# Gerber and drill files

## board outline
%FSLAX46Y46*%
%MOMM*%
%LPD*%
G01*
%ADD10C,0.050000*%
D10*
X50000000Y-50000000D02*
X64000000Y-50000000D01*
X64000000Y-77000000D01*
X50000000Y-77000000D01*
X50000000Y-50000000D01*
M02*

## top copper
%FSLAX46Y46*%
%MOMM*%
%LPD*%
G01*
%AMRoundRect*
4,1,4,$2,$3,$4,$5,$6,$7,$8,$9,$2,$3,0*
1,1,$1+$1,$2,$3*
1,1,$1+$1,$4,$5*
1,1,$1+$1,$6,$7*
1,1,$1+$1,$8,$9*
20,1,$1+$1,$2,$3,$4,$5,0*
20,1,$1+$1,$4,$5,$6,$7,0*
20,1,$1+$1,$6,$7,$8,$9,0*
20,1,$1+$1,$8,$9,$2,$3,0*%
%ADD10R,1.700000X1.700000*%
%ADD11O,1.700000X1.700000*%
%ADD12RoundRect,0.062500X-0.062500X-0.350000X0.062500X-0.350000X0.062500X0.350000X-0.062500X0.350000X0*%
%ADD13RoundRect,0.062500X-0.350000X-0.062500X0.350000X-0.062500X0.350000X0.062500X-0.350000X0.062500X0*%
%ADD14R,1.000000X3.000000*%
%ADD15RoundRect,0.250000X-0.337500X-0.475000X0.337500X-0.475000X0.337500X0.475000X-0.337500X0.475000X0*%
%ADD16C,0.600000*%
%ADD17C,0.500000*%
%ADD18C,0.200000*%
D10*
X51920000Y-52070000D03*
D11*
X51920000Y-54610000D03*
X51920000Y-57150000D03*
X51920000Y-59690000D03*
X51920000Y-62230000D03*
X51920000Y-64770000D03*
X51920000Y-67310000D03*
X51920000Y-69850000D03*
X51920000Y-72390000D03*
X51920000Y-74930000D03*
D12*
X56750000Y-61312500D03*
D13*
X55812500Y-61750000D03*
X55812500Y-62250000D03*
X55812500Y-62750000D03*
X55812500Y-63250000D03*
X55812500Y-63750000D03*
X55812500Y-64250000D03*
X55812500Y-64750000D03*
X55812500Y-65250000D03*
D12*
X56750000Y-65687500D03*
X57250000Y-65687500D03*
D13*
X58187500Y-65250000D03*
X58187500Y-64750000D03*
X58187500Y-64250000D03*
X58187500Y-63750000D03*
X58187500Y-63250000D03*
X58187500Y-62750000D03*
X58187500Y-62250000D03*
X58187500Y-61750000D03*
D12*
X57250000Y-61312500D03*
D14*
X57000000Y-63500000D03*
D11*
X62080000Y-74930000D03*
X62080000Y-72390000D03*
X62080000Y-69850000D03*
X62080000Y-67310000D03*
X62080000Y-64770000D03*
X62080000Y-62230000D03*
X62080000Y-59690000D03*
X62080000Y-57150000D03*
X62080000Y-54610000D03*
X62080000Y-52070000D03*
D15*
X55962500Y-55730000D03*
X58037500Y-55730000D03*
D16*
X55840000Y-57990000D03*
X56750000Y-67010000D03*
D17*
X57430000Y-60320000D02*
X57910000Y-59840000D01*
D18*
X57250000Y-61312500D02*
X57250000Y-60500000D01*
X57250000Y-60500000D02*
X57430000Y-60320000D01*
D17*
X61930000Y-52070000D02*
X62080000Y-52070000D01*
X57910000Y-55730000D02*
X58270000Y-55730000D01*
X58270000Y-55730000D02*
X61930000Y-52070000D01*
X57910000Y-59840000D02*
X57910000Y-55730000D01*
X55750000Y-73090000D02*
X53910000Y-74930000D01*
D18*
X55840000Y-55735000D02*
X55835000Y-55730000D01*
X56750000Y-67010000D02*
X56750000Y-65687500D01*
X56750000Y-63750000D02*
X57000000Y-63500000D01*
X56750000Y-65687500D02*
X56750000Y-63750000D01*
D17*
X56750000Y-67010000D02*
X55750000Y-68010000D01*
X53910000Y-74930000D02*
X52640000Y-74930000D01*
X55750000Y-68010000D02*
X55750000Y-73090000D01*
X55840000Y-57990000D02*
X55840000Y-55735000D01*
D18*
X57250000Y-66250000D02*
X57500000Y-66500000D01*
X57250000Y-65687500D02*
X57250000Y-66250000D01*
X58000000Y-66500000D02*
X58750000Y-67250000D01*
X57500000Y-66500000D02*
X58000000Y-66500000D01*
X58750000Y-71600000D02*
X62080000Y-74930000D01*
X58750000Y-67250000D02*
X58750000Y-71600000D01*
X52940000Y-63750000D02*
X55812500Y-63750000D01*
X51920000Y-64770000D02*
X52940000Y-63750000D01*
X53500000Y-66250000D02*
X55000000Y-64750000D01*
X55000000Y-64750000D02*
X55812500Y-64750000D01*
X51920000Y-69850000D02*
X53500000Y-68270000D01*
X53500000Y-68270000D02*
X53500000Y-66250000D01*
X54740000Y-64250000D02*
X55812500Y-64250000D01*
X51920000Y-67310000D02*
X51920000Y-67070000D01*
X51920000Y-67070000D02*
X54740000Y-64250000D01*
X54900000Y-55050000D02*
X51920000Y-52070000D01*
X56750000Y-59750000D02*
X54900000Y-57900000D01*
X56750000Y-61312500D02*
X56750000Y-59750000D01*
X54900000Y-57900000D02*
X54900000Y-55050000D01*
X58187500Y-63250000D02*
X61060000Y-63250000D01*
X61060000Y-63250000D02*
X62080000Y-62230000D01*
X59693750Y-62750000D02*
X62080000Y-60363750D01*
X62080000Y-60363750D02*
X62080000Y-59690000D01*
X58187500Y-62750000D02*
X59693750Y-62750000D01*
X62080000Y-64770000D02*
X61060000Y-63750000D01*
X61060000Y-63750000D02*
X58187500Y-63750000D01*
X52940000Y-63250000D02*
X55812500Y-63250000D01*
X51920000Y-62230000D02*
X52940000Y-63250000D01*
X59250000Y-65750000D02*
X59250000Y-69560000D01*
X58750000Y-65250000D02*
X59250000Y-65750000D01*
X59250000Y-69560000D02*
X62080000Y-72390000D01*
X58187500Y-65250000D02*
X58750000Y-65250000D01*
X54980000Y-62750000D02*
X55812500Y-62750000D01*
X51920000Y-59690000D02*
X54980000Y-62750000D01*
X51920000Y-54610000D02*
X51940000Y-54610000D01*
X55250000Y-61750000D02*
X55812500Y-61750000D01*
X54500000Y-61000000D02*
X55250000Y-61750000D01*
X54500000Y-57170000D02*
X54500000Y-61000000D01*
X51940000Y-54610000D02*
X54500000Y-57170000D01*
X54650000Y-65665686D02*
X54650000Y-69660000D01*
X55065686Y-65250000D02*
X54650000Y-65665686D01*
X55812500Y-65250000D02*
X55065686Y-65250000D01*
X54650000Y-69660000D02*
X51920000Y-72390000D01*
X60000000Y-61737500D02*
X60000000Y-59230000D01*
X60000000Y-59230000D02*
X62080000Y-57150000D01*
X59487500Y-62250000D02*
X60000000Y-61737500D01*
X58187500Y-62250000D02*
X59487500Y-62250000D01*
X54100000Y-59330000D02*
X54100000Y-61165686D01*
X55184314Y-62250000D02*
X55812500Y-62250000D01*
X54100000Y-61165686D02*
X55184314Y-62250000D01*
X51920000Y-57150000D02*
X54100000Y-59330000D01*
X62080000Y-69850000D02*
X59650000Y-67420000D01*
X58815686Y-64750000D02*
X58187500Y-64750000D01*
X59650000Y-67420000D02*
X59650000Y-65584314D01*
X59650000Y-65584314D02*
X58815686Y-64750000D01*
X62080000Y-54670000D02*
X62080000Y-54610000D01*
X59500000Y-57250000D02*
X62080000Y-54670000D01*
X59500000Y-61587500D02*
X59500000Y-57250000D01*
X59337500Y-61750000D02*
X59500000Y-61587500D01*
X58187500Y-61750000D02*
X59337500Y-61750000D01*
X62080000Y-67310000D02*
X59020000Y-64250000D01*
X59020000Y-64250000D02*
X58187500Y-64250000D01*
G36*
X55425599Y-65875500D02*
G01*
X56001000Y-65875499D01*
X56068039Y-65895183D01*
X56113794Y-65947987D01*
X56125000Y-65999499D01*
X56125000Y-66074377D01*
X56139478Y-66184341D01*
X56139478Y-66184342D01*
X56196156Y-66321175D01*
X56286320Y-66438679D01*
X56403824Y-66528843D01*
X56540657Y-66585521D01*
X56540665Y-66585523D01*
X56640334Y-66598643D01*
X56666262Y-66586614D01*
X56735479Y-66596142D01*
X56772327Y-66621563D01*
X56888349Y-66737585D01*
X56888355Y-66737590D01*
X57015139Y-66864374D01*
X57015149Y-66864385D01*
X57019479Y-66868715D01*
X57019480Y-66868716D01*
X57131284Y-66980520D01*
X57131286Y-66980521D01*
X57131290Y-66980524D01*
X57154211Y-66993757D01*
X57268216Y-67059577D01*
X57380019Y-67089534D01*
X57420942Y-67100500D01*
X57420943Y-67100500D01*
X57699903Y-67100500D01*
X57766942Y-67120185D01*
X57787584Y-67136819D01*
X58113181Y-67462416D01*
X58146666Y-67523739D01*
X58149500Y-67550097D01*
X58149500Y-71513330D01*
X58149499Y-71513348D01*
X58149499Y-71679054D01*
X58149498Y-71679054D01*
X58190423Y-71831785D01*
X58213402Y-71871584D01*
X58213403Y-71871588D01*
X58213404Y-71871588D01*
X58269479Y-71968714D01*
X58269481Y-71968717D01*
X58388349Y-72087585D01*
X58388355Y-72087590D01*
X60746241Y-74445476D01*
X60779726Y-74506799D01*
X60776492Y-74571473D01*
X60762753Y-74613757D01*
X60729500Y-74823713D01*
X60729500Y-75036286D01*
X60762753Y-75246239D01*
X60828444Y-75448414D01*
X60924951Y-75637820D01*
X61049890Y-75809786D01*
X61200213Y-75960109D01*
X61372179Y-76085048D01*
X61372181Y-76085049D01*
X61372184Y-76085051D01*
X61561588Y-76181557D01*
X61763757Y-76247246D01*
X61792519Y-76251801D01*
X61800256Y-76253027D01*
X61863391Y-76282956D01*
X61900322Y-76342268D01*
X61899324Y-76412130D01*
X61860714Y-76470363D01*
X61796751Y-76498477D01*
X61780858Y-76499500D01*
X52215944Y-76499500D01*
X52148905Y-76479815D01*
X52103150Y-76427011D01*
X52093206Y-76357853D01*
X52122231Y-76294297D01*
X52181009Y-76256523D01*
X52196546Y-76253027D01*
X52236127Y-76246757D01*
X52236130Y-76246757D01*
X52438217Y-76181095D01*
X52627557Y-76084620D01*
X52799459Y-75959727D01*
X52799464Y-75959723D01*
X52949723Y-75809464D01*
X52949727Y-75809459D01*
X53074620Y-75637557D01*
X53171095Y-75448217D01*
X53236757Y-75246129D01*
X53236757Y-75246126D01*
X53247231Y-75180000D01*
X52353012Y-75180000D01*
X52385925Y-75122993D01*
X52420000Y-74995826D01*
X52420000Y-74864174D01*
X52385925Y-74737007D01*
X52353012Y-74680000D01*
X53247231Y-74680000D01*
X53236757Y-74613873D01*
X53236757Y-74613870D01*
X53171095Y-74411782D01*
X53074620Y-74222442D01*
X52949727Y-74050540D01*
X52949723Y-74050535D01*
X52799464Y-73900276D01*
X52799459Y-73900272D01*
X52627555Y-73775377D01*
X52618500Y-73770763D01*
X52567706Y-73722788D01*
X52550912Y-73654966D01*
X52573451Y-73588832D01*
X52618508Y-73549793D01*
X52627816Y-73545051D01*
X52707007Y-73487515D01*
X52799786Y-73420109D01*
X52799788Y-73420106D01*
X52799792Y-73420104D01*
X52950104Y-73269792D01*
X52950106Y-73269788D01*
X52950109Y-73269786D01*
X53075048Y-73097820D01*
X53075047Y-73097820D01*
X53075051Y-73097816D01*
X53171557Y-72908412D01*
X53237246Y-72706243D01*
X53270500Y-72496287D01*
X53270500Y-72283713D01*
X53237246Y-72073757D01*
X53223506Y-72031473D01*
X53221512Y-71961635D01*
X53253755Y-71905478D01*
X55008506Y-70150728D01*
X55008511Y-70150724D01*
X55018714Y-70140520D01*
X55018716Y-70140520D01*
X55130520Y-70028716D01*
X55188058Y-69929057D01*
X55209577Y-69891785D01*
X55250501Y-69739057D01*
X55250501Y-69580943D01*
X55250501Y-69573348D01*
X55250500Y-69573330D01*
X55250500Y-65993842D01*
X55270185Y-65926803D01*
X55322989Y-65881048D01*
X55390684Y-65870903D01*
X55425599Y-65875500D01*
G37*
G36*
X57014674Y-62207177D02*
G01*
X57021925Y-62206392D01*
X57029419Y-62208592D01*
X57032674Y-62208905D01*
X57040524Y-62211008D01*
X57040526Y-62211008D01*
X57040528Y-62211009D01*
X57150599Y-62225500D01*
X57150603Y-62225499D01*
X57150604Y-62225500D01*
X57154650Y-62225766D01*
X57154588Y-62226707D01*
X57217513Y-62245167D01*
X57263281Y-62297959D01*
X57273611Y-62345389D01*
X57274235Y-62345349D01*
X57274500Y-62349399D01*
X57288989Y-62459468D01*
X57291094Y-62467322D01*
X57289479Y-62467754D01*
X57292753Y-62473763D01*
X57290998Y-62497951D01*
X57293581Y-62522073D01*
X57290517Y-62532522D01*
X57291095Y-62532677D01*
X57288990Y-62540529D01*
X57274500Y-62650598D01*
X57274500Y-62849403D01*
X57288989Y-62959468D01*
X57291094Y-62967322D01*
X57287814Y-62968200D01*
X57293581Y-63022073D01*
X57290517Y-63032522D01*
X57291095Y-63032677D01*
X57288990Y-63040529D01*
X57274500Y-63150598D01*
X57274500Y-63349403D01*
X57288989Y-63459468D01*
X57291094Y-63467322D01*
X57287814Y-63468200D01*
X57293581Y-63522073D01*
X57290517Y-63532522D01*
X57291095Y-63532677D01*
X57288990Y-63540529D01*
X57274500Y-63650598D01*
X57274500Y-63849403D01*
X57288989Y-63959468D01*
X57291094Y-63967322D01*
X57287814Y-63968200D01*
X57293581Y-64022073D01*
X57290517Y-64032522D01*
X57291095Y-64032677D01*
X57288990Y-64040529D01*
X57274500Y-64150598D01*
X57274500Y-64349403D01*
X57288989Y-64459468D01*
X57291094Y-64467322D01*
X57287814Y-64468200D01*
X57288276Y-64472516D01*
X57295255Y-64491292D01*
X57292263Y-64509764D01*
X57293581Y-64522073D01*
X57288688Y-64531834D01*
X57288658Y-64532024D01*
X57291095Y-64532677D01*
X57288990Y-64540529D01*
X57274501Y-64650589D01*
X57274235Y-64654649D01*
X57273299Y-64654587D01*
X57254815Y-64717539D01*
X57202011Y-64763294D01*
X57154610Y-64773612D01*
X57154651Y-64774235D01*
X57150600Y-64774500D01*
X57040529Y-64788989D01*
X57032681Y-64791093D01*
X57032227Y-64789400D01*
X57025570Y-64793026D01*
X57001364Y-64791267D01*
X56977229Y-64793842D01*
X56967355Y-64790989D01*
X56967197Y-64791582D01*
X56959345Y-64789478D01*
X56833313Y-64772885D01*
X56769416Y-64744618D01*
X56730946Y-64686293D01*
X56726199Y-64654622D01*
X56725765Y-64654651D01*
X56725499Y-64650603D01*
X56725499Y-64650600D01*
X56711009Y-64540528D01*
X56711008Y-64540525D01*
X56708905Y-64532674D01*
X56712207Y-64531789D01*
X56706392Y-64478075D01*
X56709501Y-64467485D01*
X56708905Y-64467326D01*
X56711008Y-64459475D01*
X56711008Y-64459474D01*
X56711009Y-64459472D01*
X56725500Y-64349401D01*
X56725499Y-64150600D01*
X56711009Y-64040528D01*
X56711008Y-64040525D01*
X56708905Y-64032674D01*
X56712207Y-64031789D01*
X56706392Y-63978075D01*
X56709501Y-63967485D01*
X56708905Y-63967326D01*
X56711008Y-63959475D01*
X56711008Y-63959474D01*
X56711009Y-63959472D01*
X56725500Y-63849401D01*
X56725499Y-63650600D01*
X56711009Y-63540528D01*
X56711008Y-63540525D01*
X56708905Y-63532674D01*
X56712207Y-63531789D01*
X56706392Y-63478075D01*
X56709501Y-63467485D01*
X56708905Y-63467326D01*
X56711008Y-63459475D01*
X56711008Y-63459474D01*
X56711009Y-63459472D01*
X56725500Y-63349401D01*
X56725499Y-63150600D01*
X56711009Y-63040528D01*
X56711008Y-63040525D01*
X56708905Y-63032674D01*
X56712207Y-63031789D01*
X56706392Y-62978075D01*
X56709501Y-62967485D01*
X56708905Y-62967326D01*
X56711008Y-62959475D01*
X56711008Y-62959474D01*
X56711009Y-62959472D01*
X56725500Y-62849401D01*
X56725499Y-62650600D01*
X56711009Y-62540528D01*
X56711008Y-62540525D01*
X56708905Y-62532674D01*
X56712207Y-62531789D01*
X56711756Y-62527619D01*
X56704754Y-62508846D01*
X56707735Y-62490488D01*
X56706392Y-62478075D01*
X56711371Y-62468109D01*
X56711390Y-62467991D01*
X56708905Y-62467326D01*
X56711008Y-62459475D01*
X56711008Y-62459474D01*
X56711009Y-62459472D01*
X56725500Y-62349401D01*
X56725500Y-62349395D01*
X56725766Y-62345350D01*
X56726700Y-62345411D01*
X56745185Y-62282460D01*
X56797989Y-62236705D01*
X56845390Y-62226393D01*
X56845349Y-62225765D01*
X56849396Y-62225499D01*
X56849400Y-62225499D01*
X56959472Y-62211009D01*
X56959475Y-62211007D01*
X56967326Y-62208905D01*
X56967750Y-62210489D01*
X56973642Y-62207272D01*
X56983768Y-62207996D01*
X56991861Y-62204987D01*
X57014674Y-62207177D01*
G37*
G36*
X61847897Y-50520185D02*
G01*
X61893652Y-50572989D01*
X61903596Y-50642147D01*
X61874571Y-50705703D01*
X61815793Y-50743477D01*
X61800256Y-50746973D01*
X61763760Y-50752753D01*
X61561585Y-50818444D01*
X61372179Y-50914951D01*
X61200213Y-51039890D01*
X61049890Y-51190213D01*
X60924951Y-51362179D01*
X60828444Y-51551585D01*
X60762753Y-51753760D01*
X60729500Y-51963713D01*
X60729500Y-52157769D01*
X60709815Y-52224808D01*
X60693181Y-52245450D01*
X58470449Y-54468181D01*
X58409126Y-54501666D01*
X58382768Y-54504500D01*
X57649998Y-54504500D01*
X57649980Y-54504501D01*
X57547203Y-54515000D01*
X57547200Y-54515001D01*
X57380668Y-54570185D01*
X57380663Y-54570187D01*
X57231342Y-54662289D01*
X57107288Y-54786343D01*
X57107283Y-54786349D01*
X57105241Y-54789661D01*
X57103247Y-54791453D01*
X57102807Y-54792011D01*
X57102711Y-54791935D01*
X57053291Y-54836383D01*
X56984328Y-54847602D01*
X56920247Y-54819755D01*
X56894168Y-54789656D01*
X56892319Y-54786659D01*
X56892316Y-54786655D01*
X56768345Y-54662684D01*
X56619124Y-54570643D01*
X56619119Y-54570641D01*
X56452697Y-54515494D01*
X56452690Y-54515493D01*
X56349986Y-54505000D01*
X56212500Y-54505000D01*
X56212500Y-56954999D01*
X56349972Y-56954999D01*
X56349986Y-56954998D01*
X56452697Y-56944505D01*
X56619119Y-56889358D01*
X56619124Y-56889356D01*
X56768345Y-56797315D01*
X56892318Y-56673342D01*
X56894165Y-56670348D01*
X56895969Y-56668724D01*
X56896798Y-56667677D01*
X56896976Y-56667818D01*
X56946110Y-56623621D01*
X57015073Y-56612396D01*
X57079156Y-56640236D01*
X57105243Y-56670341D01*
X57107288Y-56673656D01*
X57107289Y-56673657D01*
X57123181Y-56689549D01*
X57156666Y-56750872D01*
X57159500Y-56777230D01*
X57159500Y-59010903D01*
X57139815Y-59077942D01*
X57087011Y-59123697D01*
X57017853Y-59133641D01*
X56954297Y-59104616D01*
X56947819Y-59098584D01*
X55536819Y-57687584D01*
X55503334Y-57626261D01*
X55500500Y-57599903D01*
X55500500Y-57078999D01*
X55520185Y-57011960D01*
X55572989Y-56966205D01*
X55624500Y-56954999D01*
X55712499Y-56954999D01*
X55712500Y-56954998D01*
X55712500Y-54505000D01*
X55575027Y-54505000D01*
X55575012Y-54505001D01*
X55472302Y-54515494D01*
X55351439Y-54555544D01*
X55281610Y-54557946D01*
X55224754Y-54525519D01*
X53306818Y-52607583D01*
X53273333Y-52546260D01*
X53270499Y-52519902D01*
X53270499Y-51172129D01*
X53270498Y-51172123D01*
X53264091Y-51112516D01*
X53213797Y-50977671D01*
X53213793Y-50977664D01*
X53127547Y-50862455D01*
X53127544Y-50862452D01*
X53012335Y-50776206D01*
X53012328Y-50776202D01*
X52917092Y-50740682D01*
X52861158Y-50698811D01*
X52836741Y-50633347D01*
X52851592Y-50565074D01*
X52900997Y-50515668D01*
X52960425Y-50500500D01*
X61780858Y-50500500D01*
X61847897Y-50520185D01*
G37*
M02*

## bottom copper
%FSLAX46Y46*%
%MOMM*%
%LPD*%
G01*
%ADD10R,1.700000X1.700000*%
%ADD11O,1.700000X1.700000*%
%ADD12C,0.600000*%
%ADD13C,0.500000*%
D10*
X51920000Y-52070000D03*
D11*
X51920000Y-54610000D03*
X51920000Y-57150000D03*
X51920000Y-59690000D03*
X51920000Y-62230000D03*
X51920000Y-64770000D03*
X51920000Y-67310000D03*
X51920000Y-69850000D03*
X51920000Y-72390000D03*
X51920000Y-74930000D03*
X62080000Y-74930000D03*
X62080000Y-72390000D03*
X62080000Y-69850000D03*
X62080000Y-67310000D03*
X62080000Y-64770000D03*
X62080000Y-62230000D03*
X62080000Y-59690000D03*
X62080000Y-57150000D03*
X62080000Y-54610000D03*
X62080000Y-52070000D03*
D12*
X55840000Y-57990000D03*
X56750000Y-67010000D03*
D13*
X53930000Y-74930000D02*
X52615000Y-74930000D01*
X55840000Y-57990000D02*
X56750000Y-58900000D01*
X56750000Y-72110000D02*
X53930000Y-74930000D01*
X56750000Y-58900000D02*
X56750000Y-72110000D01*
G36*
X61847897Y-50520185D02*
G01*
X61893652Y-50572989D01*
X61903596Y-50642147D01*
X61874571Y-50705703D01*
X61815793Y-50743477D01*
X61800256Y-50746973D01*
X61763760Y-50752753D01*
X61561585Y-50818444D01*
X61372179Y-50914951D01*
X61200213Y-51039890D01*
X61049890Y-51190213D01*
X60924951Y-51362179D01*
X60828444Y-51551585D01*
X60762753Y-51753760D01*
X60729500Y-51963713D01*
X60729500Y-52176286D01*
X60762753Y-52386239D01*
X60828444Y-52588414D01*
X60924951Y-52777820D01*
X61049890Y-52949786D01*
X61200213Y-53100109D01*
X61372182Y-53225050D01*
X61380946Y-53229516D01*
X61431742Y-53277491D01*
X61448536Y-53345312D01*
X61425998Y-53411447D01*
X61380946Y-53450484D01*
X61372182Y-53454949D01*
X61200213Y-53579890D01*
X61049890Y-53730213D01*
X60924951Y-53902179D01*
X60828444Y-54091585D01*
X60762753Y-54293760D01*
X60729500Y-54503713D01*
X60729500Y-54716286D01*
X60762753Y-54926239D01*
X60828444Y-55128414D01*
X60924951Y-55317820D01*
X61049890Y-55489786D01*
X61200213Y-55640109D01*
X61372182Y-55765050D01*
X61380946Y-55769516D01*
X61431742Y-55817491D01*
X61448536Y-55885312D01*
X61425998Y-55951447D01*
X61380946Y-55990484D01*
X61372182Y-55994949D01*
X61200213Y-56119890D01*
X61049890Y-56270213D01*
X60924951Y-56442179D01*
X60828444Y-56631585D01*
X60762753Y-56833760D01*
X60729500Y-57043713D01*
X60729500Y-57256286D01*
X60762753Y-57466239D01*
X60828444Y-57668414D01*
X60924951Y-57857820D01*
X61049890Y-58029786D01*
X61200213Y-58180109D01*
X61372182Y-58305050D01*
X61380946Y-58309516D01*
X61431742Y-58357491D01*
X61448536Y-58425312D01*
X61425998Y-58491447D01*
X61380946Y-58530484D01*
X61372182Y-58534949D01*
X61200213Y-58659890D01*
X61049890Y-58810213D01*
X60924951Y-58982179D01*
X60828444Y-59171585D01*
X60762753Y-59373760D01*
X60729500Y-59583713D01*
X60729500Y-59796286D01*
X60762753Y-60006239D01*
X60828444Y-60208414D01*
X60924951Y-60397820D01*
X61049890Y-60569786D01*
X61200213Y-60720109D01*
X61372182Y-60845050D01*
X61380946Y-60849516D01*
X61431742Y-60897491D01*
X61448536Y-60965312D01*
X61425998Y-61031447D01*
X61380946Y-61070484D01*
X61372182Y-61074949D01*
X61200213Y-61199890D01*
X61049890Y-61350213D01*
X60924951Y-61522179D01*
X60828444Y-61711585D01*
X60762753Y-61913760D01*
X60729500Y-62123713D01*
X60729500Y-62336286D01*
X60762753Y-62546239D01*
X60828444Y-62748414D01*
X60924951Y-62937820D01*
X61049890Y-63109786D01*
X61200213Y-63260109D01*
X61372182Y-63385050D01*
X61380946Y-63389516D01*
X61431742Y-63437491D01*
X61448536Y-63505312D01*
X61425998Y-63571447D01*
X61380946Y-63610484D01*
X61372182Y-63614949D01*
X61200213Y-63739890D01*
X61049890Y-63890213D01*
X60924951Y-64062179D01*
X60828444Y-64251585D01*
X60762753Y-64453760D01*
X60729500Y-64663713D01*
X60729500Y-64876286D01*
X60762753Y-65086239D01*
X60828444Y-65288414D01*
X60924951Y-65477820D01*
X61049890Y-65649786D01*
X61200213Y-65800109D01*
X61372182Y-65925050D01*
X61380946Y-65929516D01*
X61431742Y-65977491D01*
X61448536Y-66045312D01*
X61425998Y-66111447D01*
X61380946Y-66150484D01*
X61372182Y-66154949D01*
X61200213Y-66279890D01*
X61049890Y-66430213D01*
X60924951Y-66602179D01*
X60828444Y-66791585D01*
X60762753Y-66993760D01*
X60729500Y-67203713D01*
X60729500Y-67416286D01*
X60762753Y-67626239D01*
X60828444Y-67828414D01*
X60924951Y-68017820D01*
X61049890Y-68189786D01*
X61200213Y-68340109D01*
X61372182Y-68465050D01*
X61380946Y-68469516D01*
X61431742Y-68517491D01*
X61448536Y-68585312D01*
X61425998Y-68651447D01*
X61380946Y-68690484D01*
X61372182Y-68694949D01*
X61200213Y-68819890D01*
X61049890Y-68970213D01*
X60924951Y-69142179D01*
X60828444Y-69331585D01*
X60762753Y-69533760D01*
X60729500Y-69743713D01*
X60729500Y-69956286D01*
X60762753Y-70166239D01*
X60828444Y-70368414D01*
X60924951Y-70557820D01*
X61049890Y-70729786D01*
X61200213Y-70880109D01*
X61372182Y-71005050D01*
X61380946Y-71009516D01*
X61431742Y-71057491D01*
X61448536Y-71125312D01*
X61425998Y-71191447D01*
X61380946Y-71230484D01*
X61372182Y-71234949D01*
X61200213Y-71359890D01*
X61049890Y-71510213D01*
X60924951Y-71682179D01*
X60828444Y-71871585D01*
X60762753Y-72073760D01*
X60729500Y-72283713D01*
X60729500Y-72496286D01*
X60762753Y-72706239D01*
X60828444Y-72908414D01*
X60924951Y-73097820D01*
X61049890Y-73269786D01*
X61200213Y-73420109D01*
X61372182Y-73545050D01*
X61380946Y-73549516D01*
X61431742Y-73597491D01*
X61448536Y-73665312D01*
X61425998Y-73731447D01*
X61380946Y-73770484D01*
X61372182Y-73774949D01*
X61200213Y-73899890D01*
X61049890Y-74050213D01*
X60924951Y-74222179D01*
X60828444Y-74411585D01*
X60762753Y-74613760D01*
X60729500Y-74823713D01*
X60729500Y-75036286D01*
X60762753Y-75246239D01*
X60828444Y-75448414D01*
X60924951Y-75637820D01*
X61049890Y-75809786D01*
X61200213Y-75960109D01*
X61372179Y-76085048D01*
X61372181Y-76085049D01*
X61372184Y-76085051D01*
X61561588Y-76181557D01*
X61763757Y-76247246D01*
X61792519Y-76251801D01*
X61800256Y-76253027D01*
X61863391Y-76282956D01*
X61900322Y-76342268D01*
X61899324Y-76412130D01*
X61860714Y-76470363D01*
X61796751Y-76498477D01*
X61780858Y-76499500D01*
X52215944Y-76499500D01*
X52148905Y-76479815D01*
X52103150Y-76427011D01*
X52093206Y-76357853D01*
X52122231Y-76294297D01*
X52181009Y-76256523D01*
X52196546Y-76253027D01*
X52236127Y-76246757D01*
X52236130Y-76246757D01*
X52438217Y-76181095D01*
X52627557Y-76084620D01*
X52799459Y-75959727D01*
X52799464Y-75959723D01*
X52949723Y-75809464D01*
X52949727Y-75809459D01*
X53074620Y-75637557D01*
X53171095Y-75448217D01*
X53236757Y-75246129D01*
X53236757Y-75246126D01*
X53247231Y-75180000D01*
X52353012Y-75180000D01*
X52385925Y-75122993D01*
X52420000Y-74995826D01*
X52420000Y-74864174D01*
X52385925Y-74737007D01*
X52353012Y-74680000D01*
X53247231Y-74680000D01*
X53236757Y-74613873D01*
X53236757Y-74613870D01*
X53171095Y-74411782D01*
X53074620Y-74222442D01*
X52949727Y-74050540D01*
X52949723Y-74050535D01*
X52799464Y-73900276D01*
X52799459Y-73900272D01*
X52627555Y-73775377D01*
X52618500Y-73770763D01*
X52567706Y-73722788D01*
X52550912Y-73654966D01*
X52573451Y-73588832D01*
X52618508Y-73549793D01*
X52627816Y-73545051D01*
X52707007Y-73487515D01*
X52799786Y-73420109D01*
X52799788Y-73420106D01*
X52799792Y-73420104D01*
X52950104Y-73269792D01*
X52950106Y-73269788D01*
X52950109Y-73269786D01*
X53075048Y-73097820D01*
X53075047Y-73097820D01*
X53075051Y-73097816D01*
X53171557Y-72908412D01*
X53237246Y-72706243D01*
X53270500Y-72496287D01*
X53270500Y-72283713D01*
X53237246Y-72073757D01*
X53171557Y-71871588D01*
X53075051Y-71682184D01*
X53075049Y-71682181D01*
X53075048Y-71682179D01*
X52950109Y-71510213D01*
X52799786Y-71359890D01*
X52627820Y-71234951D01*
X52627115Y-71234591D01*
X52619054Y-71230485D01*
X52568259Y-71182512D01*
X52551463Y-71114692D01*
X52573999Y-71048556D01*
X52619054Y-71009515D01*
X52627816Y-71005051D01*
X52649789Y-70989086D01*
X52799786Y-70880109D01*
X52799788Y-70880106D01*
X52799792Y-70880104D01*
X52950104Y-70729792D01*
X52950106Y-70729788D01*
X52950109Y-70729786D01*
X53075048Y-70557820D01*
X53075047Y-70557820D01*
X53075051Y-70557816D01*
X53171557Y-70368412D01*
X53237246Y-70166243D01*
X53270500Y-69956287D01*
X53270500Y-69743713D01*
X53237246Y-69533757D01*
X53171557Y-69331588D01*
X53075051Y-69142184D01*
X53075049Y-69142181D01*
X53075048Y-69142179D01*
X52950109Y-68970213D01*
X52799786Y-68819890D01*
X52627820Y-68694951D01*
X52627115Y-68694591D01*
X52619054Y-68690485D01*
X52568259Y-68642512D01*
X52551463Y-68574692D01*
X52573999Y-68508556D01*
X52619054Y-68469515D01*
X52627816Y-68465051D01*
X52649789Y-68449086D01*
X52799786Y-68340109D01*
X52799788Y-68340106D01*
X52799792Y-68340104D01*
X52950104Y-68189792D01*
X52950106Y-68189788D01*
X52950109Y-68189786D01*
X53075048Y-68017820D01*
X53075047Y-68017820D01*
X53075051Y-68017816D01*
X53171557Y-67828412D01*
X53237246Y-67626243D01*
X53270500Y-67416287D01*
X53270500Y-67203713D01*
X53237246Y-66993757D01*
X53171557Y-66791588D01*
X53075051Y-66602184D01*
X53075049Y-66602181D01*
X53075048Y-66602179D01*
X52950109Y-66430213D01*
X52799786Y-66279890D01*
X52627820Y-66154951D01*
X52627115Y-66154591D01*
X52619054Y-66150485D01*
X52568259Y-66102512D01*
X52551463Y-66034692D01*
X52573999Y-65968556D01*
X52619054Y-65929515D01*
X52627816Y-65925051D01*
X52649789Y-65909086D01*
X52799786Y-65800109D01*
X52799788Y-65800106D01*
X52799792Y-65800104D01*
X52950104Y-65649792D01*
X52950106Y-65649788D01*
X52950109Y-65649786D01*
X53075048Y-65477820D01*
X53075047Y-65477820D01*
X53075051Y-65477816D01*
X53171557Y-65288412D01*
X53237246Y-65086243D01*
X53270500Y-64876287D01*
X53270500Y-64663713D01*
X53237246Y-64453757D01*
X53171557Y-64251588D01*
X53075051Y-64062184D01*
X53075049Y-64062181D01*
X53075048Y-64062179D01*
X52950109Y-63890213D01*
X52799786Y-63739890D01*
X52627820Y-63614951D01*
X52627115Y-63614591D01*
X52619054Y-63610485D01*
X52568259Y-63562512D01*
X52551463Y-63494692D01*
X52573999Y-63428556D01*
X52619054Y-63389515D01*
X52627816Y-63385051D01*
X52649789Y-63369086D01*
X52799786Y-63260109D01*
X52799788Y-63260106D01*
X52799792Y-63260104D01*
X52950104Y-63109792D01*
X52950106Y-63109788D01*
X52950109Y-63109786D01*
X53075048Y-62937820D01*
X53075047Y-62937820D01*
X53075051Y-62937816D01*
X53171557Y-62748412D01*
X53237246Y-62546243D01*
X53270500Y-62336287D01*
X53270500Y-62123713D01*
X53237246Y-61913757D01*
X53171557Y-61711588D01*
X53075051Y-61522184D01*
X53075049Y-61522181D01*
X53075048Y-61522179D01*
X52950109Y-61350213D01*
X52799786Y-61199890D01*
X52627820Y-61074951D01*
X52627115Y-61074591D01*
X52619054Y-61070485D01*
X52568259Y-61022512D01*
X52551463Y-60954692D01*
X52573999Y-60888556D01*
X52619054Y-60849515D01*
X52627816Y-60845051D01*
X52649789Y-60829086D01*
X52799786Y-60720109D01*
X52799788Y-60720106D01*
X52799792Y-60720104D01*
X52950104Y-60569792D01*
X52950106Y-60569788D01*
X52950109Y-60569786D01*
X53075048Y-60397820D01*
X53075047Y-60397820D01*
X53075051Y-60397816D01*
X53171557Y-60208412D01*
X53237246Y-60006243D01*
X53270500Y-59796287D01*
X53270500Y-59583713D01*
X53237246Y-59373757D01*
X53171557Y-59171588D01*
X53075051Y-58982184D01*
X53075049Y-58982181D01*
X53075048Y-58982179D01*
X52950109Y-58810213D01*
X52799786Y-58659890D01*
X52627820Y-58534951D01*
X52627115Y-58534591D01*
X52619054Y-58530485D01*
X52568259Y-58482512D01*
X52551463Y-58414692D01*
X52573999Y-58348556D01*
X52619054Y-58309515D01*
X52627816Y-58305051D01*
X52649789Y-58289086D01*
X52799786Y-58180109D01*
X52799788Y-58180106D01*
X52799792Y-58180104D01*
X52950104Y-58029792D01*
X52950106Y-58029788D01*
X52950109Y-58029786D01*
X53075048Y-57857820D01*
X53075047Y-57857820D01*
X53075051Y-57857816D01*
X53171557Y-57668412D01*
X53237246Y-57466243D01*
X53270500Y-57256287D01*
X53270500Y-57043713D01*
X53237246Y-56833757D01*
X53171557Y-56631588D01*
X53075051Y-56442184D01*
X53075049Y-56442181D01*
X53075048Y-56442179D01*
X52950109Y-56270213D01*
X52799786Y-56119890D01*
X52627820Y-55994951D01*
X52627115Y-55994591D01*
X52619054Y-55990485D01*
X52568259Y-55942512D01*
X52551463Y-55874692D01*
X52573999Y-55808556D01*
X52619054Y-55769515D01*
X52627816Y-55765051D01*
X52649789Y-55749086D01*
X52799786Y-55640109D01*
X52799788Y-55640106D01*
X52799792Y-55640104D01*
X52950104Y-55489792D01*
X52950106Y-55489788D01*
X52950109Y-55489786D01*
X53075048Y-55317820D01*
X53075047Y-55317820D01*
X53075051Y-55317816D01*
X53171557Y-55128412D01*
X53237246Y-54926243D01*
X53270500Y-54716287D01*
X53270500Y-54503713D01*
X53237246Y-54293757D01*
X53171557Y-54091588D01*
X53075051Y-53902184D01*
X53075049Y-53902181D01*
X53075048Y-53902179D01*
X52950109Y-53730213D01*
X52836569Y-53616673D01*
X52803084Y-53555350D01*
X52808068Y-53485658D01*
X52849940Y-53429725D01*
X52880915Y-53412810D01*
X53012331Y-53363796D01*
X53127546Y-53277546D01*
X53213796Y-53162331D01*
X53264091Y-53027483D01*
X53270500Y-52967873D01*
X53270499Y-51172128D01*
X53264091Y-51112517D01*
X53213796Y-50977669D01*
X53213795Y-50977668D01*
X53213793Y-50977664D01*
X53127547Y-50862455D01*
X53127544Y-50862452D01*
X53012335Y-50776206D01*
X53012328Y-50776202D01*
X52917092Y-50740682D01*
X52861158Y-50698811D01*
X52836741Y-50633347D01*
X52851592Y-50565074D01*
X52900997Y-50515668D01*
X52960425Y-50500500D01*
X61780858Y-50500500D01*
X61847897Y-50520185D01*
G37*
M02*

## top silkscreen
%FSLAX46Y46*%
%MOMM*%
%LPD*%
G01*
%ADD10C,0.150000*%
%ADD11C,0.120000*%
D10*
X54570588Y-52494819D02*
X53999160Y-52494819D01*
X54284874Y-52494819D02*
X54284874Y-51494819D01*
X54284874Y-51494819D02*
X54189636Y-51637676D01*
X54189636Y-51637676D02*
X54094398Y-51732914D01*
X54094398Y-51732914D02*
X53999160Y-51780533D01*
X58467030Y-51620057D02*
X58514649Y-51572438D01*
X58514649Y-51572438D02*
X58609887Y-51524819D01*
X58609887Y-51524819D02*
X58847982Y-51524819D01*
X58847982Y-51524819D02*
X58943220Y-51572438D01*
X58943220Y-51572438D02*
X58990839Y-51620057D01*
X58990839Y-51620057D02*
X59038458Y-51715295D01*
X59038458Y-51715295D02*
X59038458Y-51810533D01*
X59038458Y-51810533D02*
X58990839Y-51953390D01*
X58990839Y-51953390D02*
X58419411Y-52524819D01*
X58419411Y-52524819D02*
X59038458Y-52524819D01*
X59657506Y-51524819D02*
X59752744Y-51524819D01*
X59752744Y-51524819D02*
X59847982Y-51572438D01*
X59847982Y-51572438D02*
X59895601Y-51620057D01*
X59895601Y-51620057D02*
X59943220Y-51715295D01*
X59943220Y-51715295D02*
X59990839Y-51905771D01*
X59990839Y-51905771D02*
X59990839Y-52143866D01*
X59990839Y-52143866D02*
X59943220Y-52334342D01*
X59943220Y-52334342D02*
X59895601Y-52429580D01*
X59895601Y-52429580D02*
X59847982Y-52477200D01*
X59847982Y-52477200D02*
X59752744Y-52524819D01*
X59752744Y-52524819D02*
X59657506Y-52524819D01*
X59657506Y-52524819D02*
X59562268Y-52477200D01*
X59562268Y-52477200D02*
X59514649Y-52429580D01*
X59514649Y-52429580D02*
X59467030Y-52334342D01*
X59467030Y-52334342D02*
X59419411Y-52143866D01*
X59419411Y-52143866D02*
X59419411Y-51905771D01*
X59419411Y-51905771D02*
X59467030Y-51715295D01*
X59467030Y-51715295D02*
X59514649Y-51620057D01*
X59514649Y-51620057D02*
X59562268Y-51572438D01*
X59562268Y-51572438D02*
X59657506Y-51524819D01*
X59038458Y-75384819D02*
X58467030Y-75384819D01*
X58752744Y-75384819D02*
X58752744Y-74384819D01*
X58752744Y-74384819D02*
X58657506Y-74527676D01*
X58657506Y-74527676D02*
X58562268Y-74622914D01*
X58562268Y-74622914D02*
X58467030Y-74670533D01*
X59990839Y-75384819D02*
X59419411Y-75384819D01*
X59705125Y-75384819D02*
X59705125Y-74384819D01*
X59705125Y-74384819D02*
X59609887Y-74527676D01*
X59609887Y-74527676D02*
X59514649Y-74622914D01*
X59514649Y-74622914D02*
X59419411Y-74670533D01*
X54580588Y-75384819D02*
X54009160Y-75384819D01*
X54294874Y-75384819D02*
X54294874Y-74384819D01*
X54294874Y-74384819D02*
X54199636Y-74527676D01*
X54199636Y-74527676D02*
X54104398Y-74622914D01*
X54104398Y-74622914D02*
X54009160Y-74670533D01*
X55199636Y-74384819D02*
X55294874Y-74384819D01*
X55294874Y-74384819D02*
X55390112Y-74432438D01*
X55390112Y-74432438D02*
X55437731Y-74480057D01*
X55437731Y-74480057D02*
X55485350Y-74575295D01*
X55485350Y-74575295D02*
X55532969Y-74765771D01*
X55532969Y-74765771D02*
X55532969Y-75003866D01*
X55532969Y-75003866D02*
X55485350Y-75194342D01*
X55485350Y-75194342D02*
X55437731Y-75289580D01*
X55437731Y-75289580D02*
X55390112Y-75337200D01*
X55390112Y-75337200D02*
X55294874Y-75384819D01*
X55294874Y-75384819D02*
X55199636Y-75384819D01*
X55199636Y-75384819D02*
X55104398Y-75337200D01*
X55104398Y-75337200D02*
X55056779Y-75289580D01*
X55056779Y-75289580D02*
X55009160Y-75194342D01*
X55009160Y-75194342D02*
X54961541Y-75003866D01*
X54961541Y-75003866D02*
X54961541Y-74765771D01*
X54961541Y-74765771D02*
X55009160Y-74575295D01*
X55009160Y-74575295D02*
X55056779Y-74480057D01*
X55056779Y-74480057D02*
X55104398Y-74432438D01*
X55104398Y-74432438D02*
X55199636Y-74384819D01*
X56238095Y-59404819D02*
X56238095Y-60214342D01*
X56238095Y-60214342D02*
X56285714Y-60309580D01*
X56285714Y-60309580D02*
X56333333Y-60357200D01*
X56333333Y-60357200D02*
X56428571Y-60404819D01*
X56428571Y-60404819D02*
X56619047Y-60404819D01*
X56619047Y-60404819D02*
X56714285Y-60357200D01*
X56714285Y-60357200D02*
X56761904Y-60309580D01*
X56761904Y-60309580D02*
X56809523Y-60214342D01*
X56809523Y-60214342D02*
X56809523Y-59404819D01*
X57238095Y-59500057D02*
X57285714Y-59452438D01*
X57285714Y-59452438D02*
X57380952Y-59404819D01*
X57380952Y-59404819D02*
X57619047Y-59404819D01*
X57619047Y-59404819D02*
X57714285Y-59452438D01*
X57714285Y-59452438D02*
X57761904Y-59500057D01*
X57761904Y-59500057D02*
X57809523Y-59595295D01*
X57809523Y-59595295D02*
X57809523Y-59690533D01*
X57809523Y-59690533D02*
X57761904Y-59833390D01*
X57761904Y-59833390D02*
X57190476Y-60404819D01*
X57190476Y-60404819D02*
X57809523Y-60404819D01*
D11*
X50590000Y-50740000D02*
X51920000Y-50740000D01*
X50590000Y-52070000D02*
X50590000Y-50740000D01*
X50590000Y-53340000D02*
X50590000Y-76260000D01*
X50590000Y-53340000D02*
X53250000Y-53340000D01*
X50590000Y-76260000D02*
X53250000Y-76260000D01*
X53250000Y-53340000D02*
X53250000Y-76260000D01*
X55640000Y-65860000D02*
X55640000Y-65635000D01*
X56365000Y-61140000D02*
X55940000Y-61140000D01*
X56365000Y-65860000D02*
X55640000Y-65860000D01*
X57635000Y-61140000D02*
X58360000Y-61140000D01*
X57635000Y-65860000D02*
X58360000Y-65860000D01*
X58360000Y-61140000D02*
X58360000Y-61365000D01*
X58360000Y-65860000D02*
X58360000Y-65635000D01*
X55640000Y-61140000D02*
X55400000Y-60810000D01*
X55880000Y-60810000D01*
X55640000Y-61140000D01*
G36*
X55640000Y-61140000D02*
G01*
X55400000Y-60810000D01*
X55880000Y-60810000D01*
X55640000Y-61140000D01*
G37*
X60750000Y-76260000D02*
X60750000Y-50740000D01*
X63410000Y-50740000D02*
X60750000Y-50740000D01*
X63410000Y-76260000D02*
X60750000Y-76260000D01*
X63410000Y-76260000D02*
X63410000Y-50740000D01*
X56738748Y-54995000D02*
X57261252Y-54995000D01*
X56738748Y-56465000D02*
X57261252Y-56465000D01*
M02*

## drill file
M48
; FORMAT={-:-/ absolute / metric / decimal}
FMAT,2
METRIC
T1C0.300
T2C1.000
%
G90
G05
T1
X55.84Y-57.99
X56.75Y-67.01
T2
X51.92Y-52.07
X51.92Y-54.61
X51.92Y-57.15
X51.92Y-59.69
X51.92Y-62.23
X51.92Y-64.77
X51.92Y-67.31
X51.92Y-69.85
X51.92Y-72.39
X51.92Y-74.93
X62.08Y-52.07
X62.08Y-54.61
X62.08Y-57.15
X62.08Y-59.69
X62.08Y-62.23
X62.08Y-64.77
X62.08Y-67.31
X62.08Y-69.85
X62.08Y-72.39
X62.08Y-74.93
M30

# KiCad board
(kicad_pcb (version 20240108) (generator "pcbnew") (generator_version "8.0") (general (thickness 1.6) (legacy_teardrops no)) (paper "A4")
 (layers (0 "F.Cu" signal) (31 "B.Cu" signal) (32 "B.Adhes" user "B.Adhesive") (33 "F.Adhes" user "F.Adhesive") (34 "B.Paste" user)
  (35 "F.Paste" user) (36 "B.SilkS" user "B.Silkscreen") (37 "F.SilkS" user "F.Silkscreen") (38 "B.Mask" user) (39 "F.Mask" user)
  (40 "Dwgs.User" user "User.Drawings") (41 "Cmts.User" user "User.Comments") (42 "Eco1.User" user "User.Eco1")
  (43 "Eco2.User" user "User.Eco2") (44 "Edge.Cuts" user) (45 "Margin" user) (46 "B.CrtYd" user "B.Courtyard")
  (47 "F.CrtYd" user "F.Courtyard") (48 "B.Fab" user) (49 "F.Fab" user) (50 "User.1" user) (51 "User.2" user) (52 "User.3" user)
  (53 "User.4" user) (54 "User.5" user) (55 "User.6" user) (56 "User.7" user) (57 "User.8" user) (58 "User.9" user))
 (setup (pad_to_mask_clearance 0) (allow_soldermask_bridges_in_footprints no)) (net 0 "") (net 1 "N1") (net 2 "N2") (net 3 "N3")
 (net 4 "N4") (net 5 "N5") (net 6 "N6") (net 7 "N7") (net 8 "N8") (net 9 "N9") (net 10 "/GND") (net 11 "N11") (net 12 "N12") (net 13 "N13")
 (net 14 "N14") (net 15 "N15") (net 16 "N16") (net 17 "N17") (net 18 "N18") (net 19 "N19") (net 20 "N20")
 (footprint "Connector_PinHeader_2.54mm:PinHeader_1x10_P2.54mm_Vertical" (layer "F.Cu") (at 51.92 52.07)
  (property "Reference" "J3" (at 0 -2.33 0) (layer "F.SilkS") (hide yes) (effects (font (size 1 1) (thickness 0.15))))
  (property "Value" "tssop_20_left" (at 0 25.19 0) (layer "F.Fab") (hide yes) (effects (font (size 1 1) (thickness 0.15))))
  (fp_line (start -1.33 -1.33) (end 0 -1.33) (stroke (width 0.12) (type solid)) (layer "F.SilkS"))
  (fp_line (start -1.33 0) (end -1.33 -1.33) (stroke (width 0.12) (type solid)) (layer "F.SilkS"))
  (fp_line (start -1.33 1.27) (end -1.33 24.19) (stroke (width 0.12) (type solid)) (layer "F.SilkS"))
  (fp_line (start -1.33 1.27) (end 1.33 1.27) (stroke (width 0.12) (type solid)) (layer "F.SilkS"))
  (fp_line (start -1.33 24.19) (end 1.33 24.19) (stroke (width 0.12) (type solid)) (layer "F.SilkS"))
  (fp_line (start 1.33 1.27) (end 1.33 24.19) (stroke (width 0.12) (type solid)) (layer "F.SilkS"))
  (pad "1" thru_hole rect (at 0 0) (size 1.7 1.7) (drill 1) (layers "*.Cu" "*.Mask") (remove_unused_layers no) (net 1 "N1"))
  (pad "2" thru_hole oval (at 0 2.54) (size 1.7 1.7) (drill 1) (layers "*.Cu" "*.Mask") (remove_unused_layers no) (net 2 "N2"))
  (pad "3" thru_hole oval (at 0 5.08) (size 1.7 1.7) (drill 1) (layers "*.Cu" "*.Mask") (remove_unused_layers no) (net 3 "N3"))
  (pad "4" thru_hole oval (at 0 7.62) (size 1.7 1.7) (drill 1) (layers "*.Cu" "*.Mask") (remove_unused_layers no) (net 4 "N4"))
  (pad "5" thru_hole oval (at 0 10.16) (size 1.7 1.7) (drill 1) (layers "*.Cu" "*.Mask") (remove_unused_layers no) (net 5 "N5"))
  (pad "6" thru_hole oval (at 0 12.7) (size 1.7 1.7) (drill 1) (layers "*.Cu" "*.Mask") (remove_unused_layers no) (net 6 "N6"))
  (pad "7" thru_hole oval (at 0 15.24) (size 1.7 1.7) (drill 1) (layers "*.Cu" "*.Mask") (remove_unused_layers no) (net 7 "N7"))
  (pad "8" thru_hole oval (at 0 17.78) (size 1.7 1.7) (drill 1) (layers "*.Cu" "*.Mask") (remove_unused_layers no) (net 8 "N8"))
  (pad "9" thru_hole oval (at 0 20.32) (size 1.7 1.7) (drill 1) (layers "*.Cu" "*.Mask") (remove_unused_layers no) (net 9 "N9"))
  (pad "10" thru_hole oval (at 0 22.86) (size 1.7 1.7) (drill 1) (layers "*.Cu" "*.Mask") (remove_unused_layers no) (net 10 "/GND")))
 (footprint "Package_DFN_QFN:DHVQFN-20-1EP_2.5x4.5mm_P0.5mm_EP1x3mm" (layer "F.Cu") (at 57 63.5)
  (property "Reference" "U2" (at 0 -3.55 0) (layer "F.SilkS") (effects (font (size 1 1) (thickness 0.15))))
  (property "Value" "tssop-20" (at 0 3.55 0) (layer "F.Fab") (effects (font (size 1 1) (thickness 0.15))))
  (fp_line (start -1.36 2.36) (end -1.36 2.135) (stroke (width 0.12) (type solid)) (layer "F.SilkS"))
  (fp_line (start -0.635 -2.36) (end -1.06 -2.36) (stroke (width 0.12) (type solid)) (layer "F.SilkS"))
  (fp_line (start -0.635 2.36) (end -1.36 2.36) (stroke (width 0.12) (type solid)) (layer "F.SilkS"))
  (fp_line (start 0.635 -2.36) (end 1.36 -2.36) (stroke (width 0.12) (type solid)) (layer "F.SilkS"))
  (fp_line (start 0.635 2.36) (end 1.36 2.36) (stroke (width 0.12) (type solid)) (layer "F.SilkS"))
  (fp_line (start 1.36 -2.36) (end 1.36 -2.135) (stroke (width 0.12) (type solid)) (layer "F.SilkS"))
  (fp_line (start 1.36 2.36) (end 1.36 2.135) (stroke (width 0.12) (type solid)) (layer "F.SilkS"))
  (fp_poly
   (pts (xy -1.36 -2.36) (xy -1.6 -2.69) (xy -1.12 -2.69) (xy -1.36 -2.36)) (stroke (width 0.12) (type solid)) (fill solid)
   (layer "F.SilkS"))
  (pad "" smd roundrect (at 0 -0.75) (size 0.81 1.21) (layers "F.Paste") (roundrect_rratio 0.25))
  (pad "" smd roundrect (at 0 0.75) (size 0.81 1.21) (layers "F.Paste") (roundrect_rratio 0.25))
  (pad "1" smd roundrect (at -0.25 -2.1875) (size 0.25 0.825) (layers "F.Cu" "F.Paste" "F.Mask") (roundrect_rratio 0.25) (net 1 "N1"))
  (pad "2" smd roundrect (at -1.1875 -1.75) (size 0.825 0.25) (layers "F.Cu" "F.Paste" "F.Mask") (roundrect_rratio 0.25) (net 2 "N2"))
  (pad "3" smd roundrect (at -1.1875 -1.25) (size 0.825 0.25) (layers "F.Cu" "F.Paste" "F.Mask") (roundrect_rratio 0.25) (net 3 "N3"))
  (pad "4" smd roundrect (at -1.1875 -0.75) (size 0.825 0.25) (layers "F.Cu" "F.Paste" "F.Mask") (roundrect_rratio 0.25) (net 4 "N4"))
  (pad "5" smd roundrect (at -1.1875 -0.25) (size 0.825 0.25) (layers "F.Cu" "F.Paste" "F.Mask") (roundrect_rratio 0.25) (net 5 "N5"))
  (pad "6" smd roundrect (at -1.1875 0.25) (size 0.825 0.25) (layers "F.Cu" "F.Paste" "F.Mask") (roundrect_rratio 0.25) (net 6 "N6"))
  (pad "7" smd roundrect (at -1.1875 0.75) (size 0.825 0.25) (layers "F.Cu" "F.Paste" "F.Mask") (roundrect_rratio 0.25) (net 7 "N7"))
  (pad "8" smd roundrect (at -1.1875 1.25) (size 0.825 0.25) (layers "F.Cu" "F.Paste" "F.Mask") (roundrect_rratio 0.25) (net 8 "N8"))
  (pad "9" smd roundrect (at -1.1875 1.75) (size 0.825 0.25) (layers "F.Cu" "F.Paste" "F.Mask") (roundrect_rratio 0.25) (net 9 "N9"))
  (pad "10" smd roundrect (at -0.25 2.1875) (size 0.25 0.825) (layers "F.Cu" "F.Paste" "F.Mask") (roundrect_rratio 0.25) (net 10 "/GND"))
  (pad "11" smd roundrect (at 0.25 2.1875) (size 0.25 0.825) (layers "F.Cu" "F.Paste" "F.Mask") (roundrect_rratio 0.25) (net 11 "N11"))
  (pad "12" smd roundrect (at 1.1875 1.75) (size 0.825 0.25) (layers "F.Cu" "F.Paste" "F.Mask") (roundrect_rratio 0.25) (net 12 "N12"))
  (pad "13" smd roundrect (at 1.1875 1.25) (size 0.825 0.25) (layers "F.Cu" "F.Paste" "F.Mask") (roundrect_rratio 0.25) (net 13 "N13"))
  (pad "14" smd roundrect (at 1.1875 0.75) (size 0.825 0.25) (layers "F.Cu" "F.Paste" "F.Mask") (roundrect_rratio 0.25) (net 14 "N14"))
  (pad "15" smd roundrect (at 1.1875 0.25) (size 0.825 0.25) (layers "F.Cu" "F.Paste" "F.Mask") (roundrect_rratio 0.25) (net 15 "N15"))
  (pad "16" smd roundrect (at 1.1875 -0.25) (size 0.825 0.25) (layers "F.Cu" "F.Paste" "F.Mask") (roundrect_rratio 0.25) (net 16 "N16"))
  (pad "17" smd roundrect (at 1.1875 -0.75) (size 0.825 0.25) (layers "F.Cu" "F.Paste" "F.Mask") (roundrect_rratio 0.25) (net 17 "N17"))
  (pad "18" smd roundrect (at 1.1875 -1.25) (size 0.825 0.25) (layers "F.Cu" "F.Paste" "F.Mask") (roundrect_rratio 0.25) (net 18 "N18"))
  (pad "19" smd roundrect (at 1.1875 -1.75) (size 0.825 0.25) (layers "F.Cu" "F.Paste" "F.Mask") (roundrect_rratio 0.25) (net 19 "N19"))
  (pad "20" smd roundrect (at 0.25 -2.1875) (size 0.25 0.825) (layers "F.Cu" "F.Paste" "F.Mask") (roundrect_rratio 0.25) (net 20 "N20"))
  (pad "21" smd rect (at 0 0) (size 1 3) (layers "F.Cu" "F.Mask") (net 10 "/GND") (zone_connect 2)))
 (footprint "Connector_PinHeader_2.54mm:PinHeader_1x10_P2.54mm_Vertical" (layer "F.Cu") (at 62.08 74.93 180)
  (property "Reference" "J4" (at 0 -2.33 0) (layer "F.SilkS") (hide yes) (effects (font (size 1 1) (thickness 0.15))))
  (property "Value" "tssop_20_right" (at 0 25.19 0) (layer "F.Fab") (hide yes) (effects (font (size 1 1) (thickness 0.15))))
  (fp_line (start 1.33 -1.33) (end 1.33 24.19) (stroke (width 0.12) (type solid)) (layer "F.SilkS"))
  (fp_line (start -1.33 24.19) (end 1.33 24.19) (stroke (width 0.12) (type solid)) (layer "F.SilkS"))
  (fp_line (start -1.33 -1.33) (end 1.33 -1.33) (stroke (width 0.12) (type solid)) (layer "F.SilkS"))
  (fp_line (start -1.33 -1.33) (end -1.33 24.19) (stroke (width 0.12) (type solid)) (layer "F.SilkS"))
  (pad "1" thru_hole oval (at 0 0 180) (size 1.7 1.7) (drill 1) (layers "*.Cu" "*.Mask") (remove_unused_layers no) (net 11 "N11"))
  (pad "2" thru_hole oval (at 0 2.54 180) (size 1.7 1.7) (drill 1) (layers "*.Cu" "*.Mask") (remove_unused_layers no) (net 12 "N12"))
  (pad "3" thru_hole oval (at 0 5.08 180) (size 1.7 1.7) (drill 1) (layers "*.Cu" "*.Mask") (remove_unused_layers no) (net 13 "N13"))
  (pad "4" thru_hole oval (at 0 7.62 180) (size 1.7 1.7) (drill 1) (layers "*.Cu" "*.Mask") (remove_unused_layers no) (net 14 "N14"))
  (pad "5" thru_hole oval (at 0 10.16 180) (size 1.7 1.7) (drill 1) (layers "*.Cu" "*.Mask") (remove_unused_layers no) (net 15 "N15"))
  (pad "6" thru_hole oval (at 0 12.7 180) (size 1.7 1.7) (drill 1) (layers "*.Cu" "*.Mask") (remove_unused_layers no) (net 16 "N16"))
  (pad "7" thru_hole oval (at 0 15.24 180) (size 1.7 1.7) (drill 1) (layers "*.Cu" "*.Mask") (remove_unused_layers no) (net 17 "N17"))
  (pad "8" thru_hole oval (at 0 17.78 180) (size 1.7 1.7) (drill 1) (layers "*.Cu" "*.Mask") (remove_unused_layers no) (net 18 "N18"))
  (pad "9" thru_hole oval (at 0 20.32 180) (size 1.7 1.7) (drill 1) (layers "*.Cu" "*.Mask") (remove_unused_layers no) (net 19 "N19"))
  (pad "10" thru_hole oval (at 0 22.86 180) (size 1.7 1.7) (drill 1) (layers "*.Cu" "*.Mask") (remove_unused_layers no) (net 20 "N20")))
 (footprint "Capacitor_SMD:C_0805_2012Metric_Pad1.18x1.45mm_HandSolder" (layer "F.Cu") (at 57 55.73)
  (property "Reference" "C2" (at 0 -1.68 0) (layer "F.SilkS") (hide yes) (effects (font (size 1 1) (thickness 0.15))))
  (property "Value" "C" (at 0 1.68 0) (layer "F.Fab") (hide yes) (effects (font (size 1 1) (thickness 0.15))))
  (fp_line (start -0.261252 -0.735) (end 0.261252 -0.735) (stroke (width 0.12) (type solid)) (layer "F.SilkS"))
  (fp_line (start -0.261252 0.735) (end 0.261252 0.735) (stroke (width 0.12) (type solid)) (layer "F.SilkS"))
  (pad "1" smd roundrect (at -1.0375 0) (size 1.175 1.45) (layers "F.Cu" "F.Paste" "F.Mask") (roundrect_rratio 0.212766) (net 10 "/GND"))
  (pad "2" smd roundrect (at 1.0375 0) (size 1.175 1.45) (layers "F.Cu" "F.Paste" "F.Mask") (roundrect_rratio 0.212766) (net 20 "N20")))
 (gr_rect (start 50 50) (end 64 77) (stroke (width 0.05) (type default)) (fill none) (layer "Edge.Cuts"))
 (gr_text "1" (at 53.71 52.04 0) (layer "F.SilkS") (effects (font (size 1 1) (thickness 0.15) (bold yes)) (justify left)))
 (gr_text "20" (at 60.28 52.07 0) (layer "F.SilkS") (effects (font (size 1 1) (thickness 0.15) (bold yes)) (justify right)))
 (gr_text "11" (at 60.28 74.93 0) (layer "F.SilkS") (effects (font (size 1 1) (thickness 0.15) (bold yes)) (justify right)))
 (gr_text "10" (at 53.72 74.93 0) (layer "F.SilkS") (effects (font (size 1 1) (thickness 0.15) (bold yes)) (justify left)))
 (segment (start 57.43 60.32) (end 57.91 59.84) (width 0.5) (layer "F.Cu") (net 20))
 (segment (start 57.25 61.3125) (end 57.25 60.5) (width 0.2) (layer "F.Cu") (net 20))
 (segment (start 57.25 60.5) (end 57.43 60.32) (width 0.2) (layer "F.Cu") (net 20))
 (segment (start 61.93 52.07) (end 62.08 52.07) (width 0.5) (layer "F.Cu") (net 20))
 (segment (start 57.91 55.73) (end 58.27 55.73) (width 0.5) (layer "F.Cu") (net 20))
 (segment (start 58.27 55.73) (end 61.93 52.07) (width 0.5) (layer "F.Cu") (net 20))
 (segment (start 57.91 59.84) (end 57.91 55.73) (width 0.5) (layer "F.Cu") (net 20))
 (segment (start 55.75 73.09) (end 53.91 74.93) (width 0.5) (layer "F.Cu") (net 10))
 (segment (start 55.84 55.735) (end 55.835 55.73) (width 0.2) (layer "F.Cu") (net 10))
 (segment (start 56.75 67.01) (end 56.75 65.6875) (width 0.2) (layer "F.Cu") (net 10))
 (segment (start 56.75 63.75) (end 57 63.5) (width 0.2) (layer "F.Cu") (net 10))
 (segment (start 56.75 65.6875) (end 56.75 63.75) (width 0.2) (layer "F.Cu") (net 10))
 (segment (start 56.75 67.01) (end 55.75 68.01) (width 0.5) (layer "F.Cu") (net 10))
 (segment (start 53.91 74.93) (end 52.64 74.93) (width 0.5) (layer "F.Cu") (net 10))
 (segment (start 55.75 68.01) (end 55.75 73.09) (width 0.5) (layer "F.Cu") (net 10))
 (segment (start 55.84 57.99) (end 55.84 55.735) (width 0.5) (layer "F.Cu") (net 10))
 (via (at 55.84 57.99) (size 0.6) (drill 0.3) (layers "F.Cu" "B.Cu") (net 10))
 (via (at 56.75 67.01) (size 0.6) (drill 0.3) (layers "F.Cu" "B.Cu") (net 10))
 (segment (start 53.93 74.93) (end 52.615 74.93) (width 0.5) (layer "B.Cu") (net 10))
 (segment (start 55.84 57.99) (end 56.75 58.9) (width 0.5) (layer "B.Cu") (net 10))
 (segment (start 56.75 72.11) (end 53.93 74.93) (width 0.5) (layer "B.Cu") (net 10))
 (segment (start 56.75 58.9) (end 56.75 72.11) (width 0.5) (layer "B.Cu") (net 10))
 (segment (start 57.25 66.25) (end 57.5 66.5) (width 0.2) (layer "F.Cu") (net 11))
 (segment (start 57.25 65.6875) (end 57.25 66.25) (width 0.2) (layer "F.Cu") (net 11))
 (segment (start 58 66.5) (end 58.75 67.25) (width 0.2) (layer "F.Cu") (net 11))
 (segment (start 57.5 66.5) (end 58 66.5) (width 0.2) (layer "F.Cu") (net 11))
 (segment (start 58.75 71.6) (end 62.08 74.93) (width 0.2) (layer "F.Cu") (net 11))
 (segment (start 58.75 67.25) (end 58.75 71.6) (width 0.2) (layer "F.Cu") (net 11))
 (segment (start 52.94 63.75) (end 55.8125 63.75) (width 0.2) (layer "F.Cu") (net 6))
 (segment (start 51.92 64.77) (end 52.94 63.75) (width 0.2) (layer "F.Cu") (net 6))
 (segment (start 53.5 66.25) (end 55 64.75) (width 0.2) (layer "F.Cu") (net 8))
 (segment (start 55 64.75) (end 55.8125 64.75) (width 0.2) (layer "F.Cu") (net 8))
 (segment (start 51.92 69.85) (end 53.5 68.27) (width 0.2) (layer "F.Cu") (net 8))
 (segment (start 53.5 68.27) (end 53.5 66.25) (width 0.2) (layer "F.Cu") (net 8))
 (segment (start 54.74 64.25) (end 55.8125 64.25) (width 0.2) (layer "F.Cu") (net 7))
 (segment (start 51.92 67.31) (end 51.92 67.07) (width 0.2) (layer "F.Cu") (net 7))
 (segment (start 51.92 67.07) (end 54.74 64.25) (width 0.2) (layer "F.Cu") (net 7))
 (segment (start 54.9 55.05) (end 51.92 52.07) (width 0.2) (layer "F.Cu") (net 1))
 (segment (start 56.75 59.75) (end 54.9 57.9) (width 0.2) (layer "F.Cu") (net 1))
 (segment (start 56.75 61.3125) (end 56.75 59.75) (width 0.2) (layer "F.Cu") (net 1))
 (segment (start 54.9 57.9) (end 54.9 55.05) (width 0.2) (layer "F.Cu") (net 1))
 (segment (start 58.1875 63.25) (end 61.06 63.25) (width 0.2) (layer "F.Cu") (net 16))
 (segment (start 61.06 63.25) (end 62.08 62.23) (width 0.2) (layer "F.Cu") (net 16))
 (segment (start 59.69375 62.75) (end 62.08 60.36375) (width 0.2) (layer "F.Cu") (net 17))
 (segment (start 62.08 60.36375) (end 62.08 59.69) (width 0.2) (layer "F.Cu") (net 17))
 (segment (start 58.1875 62.75) (end 59.69375 62.75) (width 0.2) (layer "F.Cu") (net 17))
 (segment (start 62.08 64.77) (end 61.06 63.75) (width 0.2) (layer "F.Cu") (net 15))
 (segment (start 61.06 63.75) (end 58.1875 63.75) (width 0.2) (layer "F.Cu") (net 15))
 (segment (start 52.94 63.25) (end 55.8125 63.25) (width 0.2) (layer "F.Cu") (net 5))
 (segment (start 51.92 62.23) (end 52.94 63.25) (width 0.2) (layer "F.Cu") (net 5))
 (segment (start 59.25 65.75) (end 59.25 69.56) (width 0.2) (layer "F.Cu") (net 12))
 (segment (start 58.75 65.25) (end 59.25 65.75) (width 0.2) (layer "F.Cu") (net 12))
 (segment (start 59.25 69.56) (end 62.08 72.39) (width 0.2) (layer "F.Cu") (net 12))
 (segment (start 58.1875 65.25) (end 58.75 65.25) (width 0.2) (layer "F.Cu") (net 12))
 (segment (start 54.98 62.75) (end 55.8125 62.75) (width 0.2) (layer "F.Cu") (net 4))
 (segment (start 51.92 59.69) (end 54.98 62.75) (width 0.2) (layer "F.Cu") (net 4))
 (segment (start 51.92 54.61) (end 51.94 54.61) (width 0.2) (layer "F.Cu") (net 2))
 (segment (start 55.25 61.75) (end 55.8125 61.75) (width 0.2) (layer "F.Cu") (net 2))
 (segment (start 54.5 61) (end 55.25 61.75) (width 0.2) (layer "F.Cu") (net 2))
 (segment (start 54.5 57.17) (end 54.5 61) (width 0.2) (layer "F.Cu") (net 2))
 (segment (start 51.94 54.61) (end 54.5 57.17) (width 0.2) (layer "F.Cu") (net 2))
 (segment (start 54.65 65.665686) (end 54.65 69.66) (width 0.2) (layer "F.Cu") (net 9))
 (segment (start 55.065686 65.25) (end 54.65 65.665686) (width 0.2) (layer "F.Cu") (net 9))
 (segment (start 55.8125 65.25) (end 55.065686 65.25) (width 0.2) (layer "F.Cu") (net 9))
 (segment (start 54.65 69.66) (end 51.92 72.39) (width 0.2) (layer "F.Cu") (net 9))
 (segment (start 60 61.7375) (end 60 59.23) (width 0.2) (layer "F.Cu") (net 18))
 (segment (start 60 59.23) (end 62.08 57.15) (width 0.2) (layer "F.Cu") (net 18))
 (segment (start 59.4875 62.25) (end 60 61.7375) (width 0.2) (layer "F.Cu") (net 18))
 (segment (start 58.1875 62.25) (end 59.4875 62.25) (width 0.2) (layer "F.Cu") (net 18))
 (segment (start 54.1 59.33) (end 54.1 61.165686) (width 0.2) (layer "F.Cu") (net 3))
 (segment (start 55.184314 62.25) (end 55.8125 62.25) (width 0.2) (layer "F.Cu") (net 3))
 (segment (start 54.1 61.165686) (end 55.184314 62.25) (width 0.2) (layer "F.Cu") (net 3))
 (segment (start 51.92 57.15) (end 54.1 59.33) (width 0.2) (layer "F.Cu") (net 3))
 (segment (start 62.08 69.85) (end 59.65 67.42) (width 0.2) (layer "F.Cu") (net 13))
 (segment (start 58.815686 64.75) (end 58.1875 64.75) (width 0.2) (layer "F.Cu") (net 13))
 (segment (start 59.65 67.42) (end 59.65 65.584314) (width 0.2) (layer "F.Cu") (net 13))
 (segment (start 59.65 65.584314) (end 58.815686 64.75) (width 0.2) (layer "F.Cu") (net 13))
 (segment (start 62.08 54.67) (end 62.08 54.61) (width 0.2) (layer "F.Cu") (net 19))
 (segment (start 59.5 57.25) (end 62.08 54.67) (width 0.2) (layer "F.Cu") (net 19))
 (segment (start 59.5 61.5875) (end 59.5 57.25) (width 0.2) (layer "F.Cu") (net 19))
 (segment (start 59.3375 61.75) (end 59.5 61.5875) (width 0.2) (layer "F.Cu") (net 19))
 (segment (start 58.1875 61.75) (end 59.3375 61.75) (width 0.2) (layer "F.Cu") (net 19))
 (segment (start 62.08 67.31) (end 59.02 64.25) (width 0.2) (layer "F.Cu") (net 14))
 (segment (start 59.02 64.25) (end 58.1875 64.25) (width 0.2) (layer "F.Cu") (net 14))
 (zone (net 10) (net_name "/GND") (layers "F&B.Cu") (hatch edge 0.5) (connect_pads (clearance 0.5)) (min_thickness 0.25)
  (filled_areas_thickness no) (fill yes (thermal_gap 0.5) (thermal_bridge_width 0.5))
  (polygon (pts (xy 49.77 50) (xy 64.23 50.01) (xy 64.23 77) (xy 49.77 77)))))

